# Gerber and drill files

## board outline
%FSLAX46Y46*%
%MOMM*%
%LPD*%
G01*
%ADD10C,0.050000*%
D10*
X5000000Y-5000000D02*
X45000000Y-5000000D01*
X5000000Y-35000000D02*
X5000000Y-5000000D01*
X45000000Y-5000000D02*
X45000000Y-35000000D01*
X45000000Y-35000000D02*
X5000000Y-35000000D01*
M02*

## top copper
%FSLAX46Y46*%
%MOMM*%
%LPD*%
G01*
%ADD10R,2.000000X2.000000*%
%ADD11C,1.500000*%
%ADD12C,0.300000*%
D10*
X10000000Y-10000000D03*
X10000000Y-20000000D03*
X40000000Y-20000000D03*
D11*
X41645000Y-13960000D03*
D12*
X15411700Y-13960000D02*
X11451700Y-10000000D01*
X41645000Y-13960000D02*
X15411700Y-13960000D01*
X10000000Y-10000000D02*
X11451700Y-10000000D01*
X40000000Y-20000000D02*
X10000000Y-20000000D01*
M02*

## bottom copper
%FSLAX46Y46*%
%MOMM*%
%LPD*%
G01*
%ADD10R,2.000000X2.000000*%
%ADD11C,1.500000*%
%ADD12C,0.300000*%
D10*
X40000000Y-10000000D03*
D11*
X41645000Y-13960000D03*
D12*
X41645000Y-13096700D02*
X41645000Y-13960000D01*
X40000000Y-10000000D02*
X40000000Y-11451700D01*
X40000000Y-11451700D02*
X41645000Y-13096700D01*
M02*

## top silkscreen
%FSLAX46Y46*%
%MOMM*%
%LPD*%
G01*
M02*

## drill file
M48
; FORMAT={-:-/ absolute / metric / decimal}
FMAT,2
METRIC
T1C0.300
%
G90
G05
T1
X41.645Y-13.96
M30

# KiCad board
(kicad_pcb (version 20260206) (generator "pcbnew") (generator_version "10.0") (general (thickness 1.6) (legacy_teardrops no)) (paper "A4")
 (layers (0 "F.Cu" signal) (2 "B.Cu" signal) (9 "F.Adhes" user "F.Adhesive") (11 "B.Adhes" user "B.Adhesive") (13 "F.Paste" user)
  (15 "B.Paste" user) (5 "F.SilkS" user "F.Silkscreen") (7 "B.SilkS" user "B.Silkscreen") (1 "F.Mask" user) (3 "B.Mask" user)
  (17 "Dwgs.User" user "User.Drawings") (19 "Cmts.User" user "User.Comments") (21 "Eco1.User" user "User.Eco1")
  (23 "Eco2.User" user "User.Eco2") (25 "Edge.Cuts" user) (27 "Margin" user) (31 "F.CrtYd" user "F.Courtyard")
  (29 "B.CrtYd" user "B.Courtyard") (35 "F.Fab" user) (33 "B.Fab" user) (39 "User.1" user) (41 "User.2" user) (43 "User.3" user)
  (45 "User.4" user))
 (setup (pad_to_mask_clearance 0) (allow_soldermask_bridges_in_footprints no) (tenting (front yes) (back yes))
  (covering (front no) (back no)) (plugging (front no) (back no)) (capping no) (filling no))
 (gr_line (start 5 5) (end 45 5) (stroke (width 0.05) (type default)) (layer "Edge.Cuts"))
 (gr_line (start 5 35) (end 5 5) (stroke (width 0.05) (type default)) (layer "Edge.Cuts"))
 (gr_line (start 45 5) (end 45 35) (stroke (width 0.05) (type default)) (layer "Edge.Cuts"))
 (gr_line (start 45 35) (end 5 35) (stroke (width 0.05) (type default)) (layer "Edge.Cuts"))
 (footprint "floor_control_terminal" (layer "F.Cu") (at 10 10)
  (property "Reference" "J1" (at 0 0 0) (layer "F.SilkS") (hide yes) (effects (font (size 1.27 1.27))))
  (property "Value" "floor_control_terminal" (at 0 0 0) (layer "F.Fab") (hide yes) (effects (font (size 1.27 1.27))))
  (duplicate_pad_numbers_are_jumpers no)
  (pad "1" smd rect (at 0 0) (size 2 2) (layers "F.Cu" "F.Paste" "F.Mask") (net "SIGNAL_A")))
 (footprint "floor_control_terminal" (layer "B.Cu") (at 40 10)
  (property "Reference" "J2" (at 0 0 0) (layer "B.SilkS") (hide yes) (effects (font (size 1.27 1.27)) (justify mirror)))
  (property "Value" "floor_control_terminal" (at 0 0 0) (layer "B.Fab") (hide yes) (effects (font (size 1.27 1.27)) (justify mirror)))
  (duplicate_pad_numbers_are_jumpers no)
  (pad "1" smd rect (at 0 0) (size 2 2) (layers "B.Cu" "B.Paste" "B.Mask") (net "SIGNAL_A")))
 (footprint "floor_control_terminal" (layer "F.Cu") (at 10 20)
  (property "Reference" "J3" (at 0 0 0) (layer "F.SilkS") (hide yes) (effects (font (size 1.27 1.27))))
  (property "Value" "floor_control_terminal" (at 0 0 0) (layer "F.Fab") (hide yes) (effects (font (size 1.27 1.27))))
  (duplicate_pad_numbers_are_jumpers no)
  (pad "1" smd rect (at 0 0) (size 2 2) (layers "F.Cu" "F.Paste" "F.Mask") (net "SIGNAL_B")))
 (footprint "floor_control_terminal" (layer "F.Cu") (at 40 20)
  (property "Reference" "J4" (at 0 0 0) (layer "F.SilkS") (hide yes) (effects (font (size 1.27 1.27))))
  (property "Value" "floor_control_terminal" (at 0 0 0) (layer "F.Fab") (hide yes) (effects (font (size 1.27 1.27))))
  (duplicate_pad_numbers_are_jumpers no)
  (pad "1" smd rect (at 0 0) (size 2 2) (layers "F.Cu" "F.Paste" "F.Mask") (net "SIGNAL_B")))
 (segment (start 15.4117 13.96) (end 11.4517 10) (width 0.3) (layer "F.Cu") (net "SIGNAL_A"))
 (segment (start 41.645 13.96) (end 15.4117 13.96) (width 0.3) (layer "F.Cu") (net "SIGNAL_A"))
 (segment (start 10 10) (end 11.4517 10) (width 0.3) (layer "F.Cu") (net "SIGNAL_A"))
 (via (at 41.645 13.96) (size 1.5) (drill 0.3) (layers "F.Cu" "B.Cu") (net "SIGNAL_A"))
 (segment (start 41.645 13.0967) (end 41.645 13.96) (width 0.3) (layer "B.Cu") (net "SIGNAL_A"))
 (segment (start 40 10) (end 40 11.4517) (width 0.3) (layer "B.Cu") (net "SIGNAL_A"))
 (segment (start 40 11.4517) (end 41.645 13.0967) (width 0.3) (layer "B.Cu") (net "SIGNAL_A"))
 (segment (start 40 20) (end 10 20) (width 0.3) (layer "F.Cu") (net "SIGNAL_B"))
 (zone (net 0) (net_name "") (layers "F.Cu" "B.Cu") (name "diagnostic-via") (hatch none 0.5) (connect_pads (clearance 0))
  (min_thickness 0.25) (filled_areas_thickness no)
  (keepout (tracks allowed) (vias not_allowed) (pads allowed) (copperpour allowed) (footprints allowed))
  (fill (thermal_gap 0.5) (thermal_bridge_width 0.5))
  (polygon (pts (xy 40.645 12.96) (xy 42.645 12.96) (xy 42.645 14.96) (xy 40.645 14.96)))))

